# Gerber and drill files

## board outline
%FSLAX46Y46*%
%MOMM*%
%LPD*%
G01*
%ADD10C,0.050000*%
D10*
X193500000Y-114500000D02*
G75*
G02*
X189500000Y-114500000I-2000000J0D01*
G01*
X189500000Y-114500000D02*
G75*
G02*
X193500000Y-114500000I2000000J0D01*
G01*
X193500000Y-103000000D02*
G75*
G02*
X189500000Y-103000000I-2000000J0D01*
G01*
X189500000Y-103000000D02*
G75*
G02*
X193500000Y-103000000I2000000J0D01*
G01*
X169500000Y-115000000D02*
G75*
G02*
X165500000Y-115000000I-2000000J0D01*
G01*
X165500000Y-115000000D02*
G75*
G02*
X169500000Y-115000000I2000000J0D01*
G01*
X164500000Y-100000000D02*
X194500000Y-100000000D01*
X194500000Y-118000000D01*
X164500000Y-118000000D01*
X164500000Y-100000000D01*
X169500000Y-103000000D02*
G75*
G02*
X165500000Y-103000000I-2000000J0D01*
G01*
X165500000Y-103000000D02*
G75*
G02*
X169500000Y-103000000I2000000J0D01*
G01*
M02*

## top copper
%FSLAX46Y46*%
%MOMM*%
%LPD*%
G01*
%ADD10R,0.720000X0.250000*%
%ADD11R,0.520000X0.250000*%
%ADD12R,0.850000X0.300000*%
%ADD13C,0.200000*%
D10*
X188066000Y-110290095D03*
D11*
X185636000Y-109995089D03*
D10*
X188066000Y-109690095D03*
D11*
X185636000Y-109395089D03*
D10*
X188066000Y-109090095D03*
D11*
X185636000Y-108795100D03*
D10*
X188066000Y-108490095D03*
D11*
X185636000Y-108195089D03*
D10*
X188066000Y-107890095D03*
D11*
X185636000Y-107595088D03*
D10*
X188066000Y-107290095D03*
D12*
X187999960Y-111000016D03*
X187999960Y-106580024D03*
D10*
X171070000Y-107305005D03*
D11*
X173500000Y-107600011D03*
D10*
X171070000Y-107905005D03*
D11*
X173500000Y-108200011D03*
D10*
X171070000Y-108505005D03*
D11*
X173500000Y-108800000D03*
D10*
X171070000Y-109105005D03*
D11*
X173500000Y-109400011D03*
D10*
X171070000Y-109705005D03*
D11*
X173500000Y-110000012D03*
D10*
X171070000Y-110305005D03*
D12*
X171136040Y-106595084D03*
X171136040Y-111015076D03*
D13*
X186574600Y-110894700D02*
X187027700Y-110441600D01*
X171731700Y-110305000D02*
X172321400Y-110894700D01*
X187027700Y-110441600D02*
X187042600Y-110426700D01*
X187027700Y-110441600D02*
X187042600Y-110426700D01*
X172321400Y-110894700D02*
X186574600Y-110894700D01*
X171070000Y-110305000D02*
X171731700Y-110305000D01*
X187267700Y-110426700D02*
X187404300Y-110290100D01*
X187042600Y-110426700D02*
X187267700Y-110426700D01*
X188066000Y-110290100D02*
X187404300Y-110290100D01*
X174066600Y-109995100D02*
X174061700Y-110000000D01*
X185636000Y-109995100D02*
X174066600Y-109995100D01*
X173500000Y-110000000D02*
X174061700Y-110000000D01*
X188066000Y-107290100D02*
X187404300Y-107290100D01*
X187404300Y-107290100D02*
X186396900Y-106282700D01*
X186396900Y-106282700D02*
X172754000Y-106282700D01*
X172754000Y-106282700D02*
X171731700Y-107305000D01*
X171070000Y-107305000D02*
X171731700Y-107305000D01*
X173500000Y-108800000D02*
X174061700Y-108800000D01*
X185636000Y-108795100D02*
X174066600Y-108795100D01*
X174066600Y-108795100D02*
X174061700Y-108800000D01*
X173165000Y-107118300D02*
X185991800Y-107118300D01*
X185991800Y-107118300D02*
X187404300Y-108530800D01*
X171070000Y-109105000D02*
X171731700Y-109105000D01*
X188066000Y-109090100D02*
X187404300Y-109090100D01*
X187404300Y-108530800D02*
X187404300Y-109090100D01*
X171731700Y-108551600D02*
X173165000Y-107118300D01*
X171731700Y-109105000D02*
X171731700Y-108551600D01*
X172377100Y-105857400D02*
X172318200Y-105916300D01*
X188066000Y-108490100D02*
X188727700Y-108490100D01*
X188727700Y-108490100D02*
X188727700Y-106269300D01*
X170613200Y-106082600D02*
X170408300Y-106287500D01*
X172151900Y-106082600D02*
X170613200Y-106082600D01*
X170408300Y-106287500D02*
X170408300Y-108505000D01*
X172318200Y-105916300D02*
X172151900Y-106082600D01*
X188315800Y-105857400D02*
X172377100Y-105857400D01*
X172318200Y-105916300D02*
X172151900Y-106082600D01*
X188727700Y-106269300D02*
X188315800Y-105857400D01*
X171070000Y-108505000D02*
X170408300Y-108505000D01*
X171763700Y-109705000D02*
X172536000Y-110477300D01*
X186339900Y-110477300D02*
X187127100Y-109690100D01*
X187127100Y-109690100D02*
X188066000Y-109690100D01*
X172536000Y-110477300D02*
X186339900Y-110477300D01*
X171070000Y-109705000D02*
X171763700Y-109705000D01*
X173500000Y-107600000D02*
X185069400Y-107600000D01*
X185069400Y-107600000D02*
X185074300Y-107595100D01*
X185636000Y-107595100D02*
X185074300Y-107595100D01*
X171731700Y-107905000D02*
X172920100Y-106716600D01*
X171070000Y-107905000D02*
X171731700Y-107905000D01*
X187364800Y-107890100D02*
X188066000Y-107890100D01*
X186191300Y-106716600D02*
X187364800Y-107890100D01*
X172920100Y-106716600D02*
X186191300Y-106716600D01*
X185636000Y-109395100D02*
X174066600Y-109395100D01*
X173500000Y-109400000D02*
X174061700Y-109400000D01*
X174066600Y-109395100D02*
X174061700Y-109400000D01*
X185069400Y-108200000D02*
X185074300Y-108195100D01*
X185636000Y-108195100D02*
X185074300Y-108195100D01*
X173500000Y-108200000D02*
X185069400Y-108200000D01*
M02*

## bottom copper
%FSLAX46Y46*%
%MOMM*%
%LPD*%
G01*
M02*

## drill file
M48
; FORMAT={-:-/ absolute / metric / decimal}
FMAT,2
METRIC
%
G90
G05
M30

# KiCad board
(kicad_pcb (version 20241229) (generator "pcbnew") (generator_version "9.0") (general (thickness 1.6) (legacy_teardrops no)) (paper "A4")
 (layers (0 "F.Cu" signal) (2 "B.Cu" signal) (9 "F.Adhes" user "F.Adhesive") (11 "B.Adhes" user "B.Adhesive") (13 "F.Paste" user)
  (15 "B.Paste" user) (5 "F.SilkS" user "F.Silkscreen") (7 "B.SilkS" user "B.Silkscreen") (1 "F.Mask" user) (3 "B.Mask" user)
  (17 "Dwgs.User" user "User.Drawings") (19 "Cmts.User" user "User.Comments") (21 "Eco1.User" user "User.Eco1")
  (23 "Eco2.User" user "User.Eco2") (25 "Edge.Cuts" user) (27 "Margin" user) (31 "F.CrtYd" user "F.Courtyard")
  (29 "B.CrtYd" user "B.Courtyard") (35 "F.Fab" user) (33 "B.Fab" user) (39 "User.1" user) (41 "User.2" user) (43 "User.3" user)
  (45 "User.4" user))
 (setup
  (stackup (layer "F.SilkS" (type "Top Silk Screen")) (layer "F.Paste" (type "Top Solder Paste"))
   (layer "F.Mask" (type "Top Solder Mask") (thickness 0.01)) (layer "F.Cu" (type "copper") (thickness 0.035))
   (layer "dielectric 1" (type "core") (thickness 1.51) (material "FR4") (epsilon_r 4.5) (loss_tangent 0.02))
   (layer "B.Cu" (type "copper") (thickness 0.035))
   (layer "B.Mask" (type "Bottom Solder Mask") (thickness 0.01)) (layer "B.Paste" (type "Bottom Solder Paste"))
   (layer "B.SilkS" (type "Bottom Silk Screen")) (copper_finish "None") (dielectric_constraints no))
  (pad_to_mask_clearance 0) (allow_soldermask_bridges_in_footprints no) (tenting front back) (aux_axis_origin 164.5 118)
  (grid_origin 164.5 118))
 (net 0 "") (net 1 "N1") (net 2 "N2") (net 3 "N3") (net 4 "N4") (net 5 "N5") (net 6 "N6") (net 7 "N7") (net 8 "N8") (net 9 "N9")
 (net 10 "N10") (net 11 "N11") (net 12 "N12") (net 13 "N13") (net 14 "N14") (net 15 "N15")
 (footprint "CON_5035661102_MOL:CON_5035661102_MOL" (layer "F.Cu") (at 186.946 108.7951 90)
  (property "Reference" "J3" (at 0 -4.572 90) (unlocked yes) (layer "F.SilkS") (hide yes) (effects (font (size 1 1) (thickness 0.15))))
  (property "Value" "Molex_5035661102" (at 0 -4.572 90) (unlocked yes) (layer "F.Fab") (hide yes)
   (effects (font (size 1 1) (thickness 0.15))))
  (pad "1" smd rect (at -1.494995 1.12 90) (size 0.25 0.72) (layers "F.Cu" "F.Mask" "F.Paste") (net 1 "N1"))
  (pad "2" smd rect (at -1.199989 -1.31 90) (size 0.25 0.52) (layers "F.Cu" "F.Mask" "F.Paste") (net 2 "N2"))
  (pad "3" smd rect (at -0.894995 1.12 90) (size 0.25 0.72) (layers "F.Cu" "F.Mask" "F.Paste") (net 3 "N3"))
  (pad "4" smd rect (at -0.599989 -1.31 90) (size 0.25 0.52) (layers "F.Cu" "F.Mask" "F.Paste") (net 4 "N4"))
  (pad "5" smd rect (at -0.294995 1.12 90) (size 0.25 0.72) (layers "F.Cu" "F.Mask" "F.Paste") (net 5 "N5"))
  (pad "6" smd rect (at 0 -1.31 90) (size 0.25 0.52) (layers "F.Cu" "F.Mask" "F.Paste") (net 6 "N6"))
  (pad "7" smd rect (at 0.305005 1.12 90) (size 0.25 0.72) (layers "F.Cu" "F.Mask" "F.Paste") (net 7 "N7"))
  (pad "8" smd rect (at 0.600011 -1.31 90) (size 0.25 0.52) (layers "F.Cu" "F.Mask" "F.Paste") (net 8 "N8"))
  (pad "9" smd rect (at 0.905005 1.12 90) (size 0.25 0.72) (layers "F.Cu" "F.Mask" "F.Paste") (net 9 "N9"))
  (pad "10" smd rect (at 1.200012 -1.31 90) (size 0.25 0.52) (layers "F.Cu" "F.Mask" "F.Paste") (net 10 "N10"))
  (pad "11" smd rect (at 1.505005 1.12 90) (size 0.25 0.72) (layers "F.Cu" "F.Mask" "F.Paste") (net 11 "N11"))
  (pad "P1" smd rect (at -2.204916 1.05396 90) (size 0.3 0.85) (layers "F.Cu" "F.Mask" "F.Paste") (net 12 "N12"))
  (pad "P2" smd rect (at 2.215076 1.05396 90) (size 0.3 0.85) (layers "F.Cu" "F.Mask" "F.Paste") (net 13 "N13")))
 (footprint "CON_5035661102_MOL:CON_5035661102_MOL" (layer "F.Cu") (at 172.19 108.8 -90)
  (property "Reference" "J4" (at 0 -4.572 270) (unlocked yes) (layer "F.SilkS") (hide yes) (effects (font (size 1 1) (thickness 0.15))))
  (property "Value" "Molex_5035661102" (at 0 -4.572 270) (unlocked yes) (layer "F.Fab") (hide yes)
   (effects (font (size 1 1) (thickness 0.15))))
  (pad "1" smd rect (at -1.494995 1.12 270) (size 0.25 0.72) (layers "F.Cu" "F.Mask" "F.Paste") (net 11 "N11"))
  (pad "2" smd rect (at -1.199989 -1.31 270) (size 0.25 0.52) (layers "F.Cu" "F.Mask" "F.Paste") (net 10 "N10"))
  (pad "3" smd rect (at -0.894995 1.12 270) (size 0.25 0.72) (layers "F.Cu" "F.Mask" "F.Paste") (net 9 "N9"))
  (pad "4" smd rect (at -0.599989 -1.31 270) (size 0.25 0.52) (layers "F.Cu" "F.Mask" "F.Paste") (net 8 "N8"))
  (pad "5" smd rect (at -0.294995 1.12 270) (size 0.25 0.72) (layers "F.Cu" "F.Mask" "F.Paste") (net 7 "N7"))
  (pad "6" smd rect (at 0 -1.31 270) (size 0.25 0.52) (layers "F.Cu" "F.Mask" "F.Paste") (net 6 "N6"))
  (pad "7" smd rect (at 0.305005 1.12 270) (size 0.25 0.72) (layers "F.Cu" "F.Mask" "F.Paste") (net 5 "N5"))
  (pad "8" smd rect (at 0.600011 -1.31 270) (size 0.25 0.52) (layers "F.Cu" "F.Mask" "F.Paste") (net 4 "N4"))
  (pad "9" smd rect (at 0.905005 1.12 270) (size 0.25 0.72) (layers "F.Cu" "F.Mask" "F.Paste") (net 3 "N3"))
  (pad "10" smd rect (at 1.200012 -1.31 270) (size 0.25 0.52) (layers "F.Cu" "F.Mask" "F.Paste") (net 2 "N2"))
  (pad "11" smd rect (at 1.505005 1.12 270) (size 0.25 0.72) (layers "F.Cu" "F.Mask" "F.Paste") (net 1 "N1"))
  (pad "P1" smd rect (at -2.204916 1.05396 270) (size 0.3 0.85) (layers "F.Cu" "F.Mask" "F.Paste") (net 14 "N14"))
  (pad "P2" smd rect (at 2.215076 1.05396 270) (size 0.3 0.85) (layers "F.Cu" "F.Mask" "F.Paste") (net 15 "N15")))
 (gr_circle (center 191.5 114.5) (end 193.5 114.5) (stroke (width 0.05) (type default)) (fill no) (layer "Edge.Cuts"))
 (gr_circle (center 191.5 103) (end 193.5 103) (stroke (width 0.05) (type default)) (fill no) (layer "Edge.Cuts"))
 (gr_circle (center 167.5 115) (end 169.5 115) (stroke (width 0.05) (type default)) (fill no) (layer "Edge.Cuts"))
 (gr_rect (start 164.5 100) (end 194.5 118) (stroke (width 0.05) (type default)) (fill no) (layer "Edge.Cuts"))
 (gr_circle (center 167.5 103) (end 169.5 103) (stroke (width 0.05) (type solid)) (fill no) (layer "Edge.Cuts"))
 (segment (start 186.5746 110.8947) (end 187.0277 110.4416) (width 0.2) (layer "F.Cu") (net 1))
 (segment (start 171.7317 110.305) (end 172.3214 110.8947) (width 0.2) (layer "F.Cu") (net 1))
 (segment (start 187.0277 110.4416) (end 187.0426 110.4267) (width 0.2) (layer "F.Cu") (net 1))
 (segment (start 187.0277 110.4416) (end 187.0426 110.4267) (width 0.2) (layer "F.Cu") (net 1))
 (segment (start 172.3214 110.8947) (end 186.5746 110.8947) (width 0.2) (layer "F.Cu") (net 1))
 (segment (start 171.07 110.305) (end 171.7317 110.305) (width 0.2) (layer "F.Cu") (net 1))
 (segment (start 187.2677 110.4267) (end 187.4043 110.2901) (width 0.2) (layer "F.Cu") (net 1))
 (segment (start 187.0426 110.4267) (end 187.2677 110.4267) (width 0.2) (layer "F.Cu") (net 1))
 (segment (start 188.066 110.2901) (end 187.4043 110.2901) (width 0.2) (layer "F.Cu") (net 1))
 (segment (start 174.0666 109.9951) (end 174.0617 110) (width 0.2) (layer "F.Cu") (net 2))
 (segment (start 185.636 109.9951) (end 174.0666 109.9951) (width 0.2) (layer "F.Cu") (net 2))
 (segment (start 173.5 110) (end 174.0617 110) (width 0.2) (layer "F.Cu") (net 2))
 (segment (start 188.066 107.2901) (end 187.4043 107.2901) (width 0.2) (layer "F.Cu") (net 11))
 (segment (start 187.4043 107.2901) (end 186.3969 106.2827) (width 0.2) (layer "F.Cu") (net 11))
 (segment (start 186.3969 106.2827) (end 172.754 106.2827) (width 0.2) (layer "F.Cu") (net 11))
 (segment (start 172.754 106.2827) (end 171.7317 107.305) (width 0.2) (layer "F.Cu") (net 11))
 (segment (start 171.07 107.305) (end 171.7317 107.305) (width 0.2) (layer "F.Cu") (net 11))
 (segment (start 173.5 108.8) (end 174.0617 108.8) (width 0.2) (layer "F.Cu") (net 6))
 (segment (start 185.636 108.7951) (end 174.0666 108.7951) (width 0.2) (layer "F.Cu") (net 6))
 (segment (start 174.0666 108.7951) (end 174.0617 108.8) (width 0.2) (layer "F.Cu") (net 6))
 (segment (start 173.165 107.1183) (end 185.9918 107.1183) (width 0.2) (layer "F.Cu") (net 5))
 (segment (start 185.9918 107.1183) (end 187.4043 108.5308) (width 0.2) (layer "F.Cu") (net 5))
 (segment (start 171.07 109.105) (end 171.7317 109.105) (width 0.2) (layer "F.Cu") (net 5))
 (segment (start 188.066 109.0901) (end 187.4043 109.0901) (width 0.2) (layer "F.Cu") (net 5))
 (segment (start 187.4043 108.5308) (end 187.4043 109.0901) (width 0.2) (layer "F.Cu") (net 5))
 (segment (start 171.7317 108.5516) (end 173.165 107.1183) (width 0.2) (layer "F.Cu") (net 5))
 (segment (start 171.7317 109.105) (end 171.7317 108.5516) (width 0.2) (layer "F.Cu") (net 5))
 (segment (start 172.3771 105.8574) (end 172.3182 105.9163) (width 0.2) (layer "F.Cu") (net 7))
 (segment (start 188.066 108.4901) (end 188.7277 108.4901) (width 0.2) (layer "F.Cu") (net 7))
 (segment (start 188.7277 108.4901) (end 188.7277 106.2693) (width 0.2) (layer "F.Cu") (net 7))
 (segment (start 170.6132 106.0826) (end 170.4083 106.2875) (width 0.2) (layer "F.Cu") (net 7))
 (segment (start 172.1519 106.0826) (end 170.6132 106.0826) (width 0.2) (layer "F.Cu") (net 7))
 (segment (start 170.4083 106.2875) (end 170.4083 108.505) (width 0.2) (layer "F.Cu") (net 7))
 (segment (start 172.3182 105.9163) (end 172.1519 106.0826) (width 0.2) (layer "F.Cu") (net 7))
 (segment (start 188.3158 105.8574) (end 172.3771 105.8574) (width 0.2) (layer "F.Cu") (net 7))
 (segment (start 172.3182 105.9163) (end 172.1519 106.0826) (width 0.2) (layer "F.Cu") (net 7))
 (segment (start 188.7277 106.2693) (end 188.3158 105.8574) (width 0.2) (layer "F.Cu") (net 7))
 (segment (start 171.07 108.505) (end 170.4083 108.505) (width 0.2) (layer "F.Cu") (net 7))
 (segment (start 171.7637 109.705) (end 172.536 110.4773) (width 0.2) (layer "F.Cu") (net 3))
 (segment (start 186.3399 110.4773) (end 187.1271 109.6901) (width 0.2) (layer "F.Cu") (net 3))
 (segment (start 187.1271 109.6901) (end 188.066 109.6901) (width 0.2) (layer "F.Cu") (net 3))
 (segment (start 172.536 110.4773) (end 186.3399 110.4773) (width 0.2) (layer "F.Cu") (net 3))
 (segment (start 171.07 109.705) (end 171.7637 109.705) (width 0.2) (layer "F.Cu") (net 3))
 (segment (start 173.5 107.6) (end 185.0694 107.6) (width 0.2) (layer "F.Cu") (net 10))
 (segment (start 185.0694 107.6) (end 185.0743 107.5951) (width 0.2) (layer "F.Cu") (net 10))
 (segment (start 185.636 107.5951) (end 185.0743 107.5951) (width 0.2) (layer "F.Cu") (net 10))
 (segment (start 171.7317 107.905) (end 172.9201 106.7166) (width 0.2) (layer "F.Cu") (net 9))
 (segment (start 171.07 107.905) (end 171.7317 107.905) (width 0.2) (layer "F.Cu") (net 9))
 (segment (start 187.3648 107.8901) (end 188.066 107.8901) (width 0.2) (layer "F.Cu") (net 9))
 (segment (start 186.1913 106.7166) (end 187.3648 107.8901) (width 0.2) (layer "F.Cu") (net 9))
 (segment (start 172.9201 106.7166) (end 186.1913 106.7166) (width 0.2) (layer "F.Cu") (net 9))
 (segment (start 185.636 109.3951) (end 174.0666 109.3951) (width 0.2) (layer "F.Cu") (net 4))
 (segment (start 173.5 109.4) (end 174.0617 109.4) (width 0.2) (layer "F.Cu") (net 4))
 (segment (start 174.0666 109.3951) (end 174.0617 109.4) (width 0.2) (layer "F.Cu") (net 4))
 (segment (start 185.0694 108.2) (end 185.0743 108.1951) (width 0.2) (layer "F.Cu") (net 8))
 (segment (start 185.636 108.1951) (end 185.0743 108.1951) (width 0.2) (layer "F.Cu") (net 8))
 (segment (start 173.5 108.2) (end 185.0694 108.2) (width 0.2) (layer "F.Cu") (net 8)))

